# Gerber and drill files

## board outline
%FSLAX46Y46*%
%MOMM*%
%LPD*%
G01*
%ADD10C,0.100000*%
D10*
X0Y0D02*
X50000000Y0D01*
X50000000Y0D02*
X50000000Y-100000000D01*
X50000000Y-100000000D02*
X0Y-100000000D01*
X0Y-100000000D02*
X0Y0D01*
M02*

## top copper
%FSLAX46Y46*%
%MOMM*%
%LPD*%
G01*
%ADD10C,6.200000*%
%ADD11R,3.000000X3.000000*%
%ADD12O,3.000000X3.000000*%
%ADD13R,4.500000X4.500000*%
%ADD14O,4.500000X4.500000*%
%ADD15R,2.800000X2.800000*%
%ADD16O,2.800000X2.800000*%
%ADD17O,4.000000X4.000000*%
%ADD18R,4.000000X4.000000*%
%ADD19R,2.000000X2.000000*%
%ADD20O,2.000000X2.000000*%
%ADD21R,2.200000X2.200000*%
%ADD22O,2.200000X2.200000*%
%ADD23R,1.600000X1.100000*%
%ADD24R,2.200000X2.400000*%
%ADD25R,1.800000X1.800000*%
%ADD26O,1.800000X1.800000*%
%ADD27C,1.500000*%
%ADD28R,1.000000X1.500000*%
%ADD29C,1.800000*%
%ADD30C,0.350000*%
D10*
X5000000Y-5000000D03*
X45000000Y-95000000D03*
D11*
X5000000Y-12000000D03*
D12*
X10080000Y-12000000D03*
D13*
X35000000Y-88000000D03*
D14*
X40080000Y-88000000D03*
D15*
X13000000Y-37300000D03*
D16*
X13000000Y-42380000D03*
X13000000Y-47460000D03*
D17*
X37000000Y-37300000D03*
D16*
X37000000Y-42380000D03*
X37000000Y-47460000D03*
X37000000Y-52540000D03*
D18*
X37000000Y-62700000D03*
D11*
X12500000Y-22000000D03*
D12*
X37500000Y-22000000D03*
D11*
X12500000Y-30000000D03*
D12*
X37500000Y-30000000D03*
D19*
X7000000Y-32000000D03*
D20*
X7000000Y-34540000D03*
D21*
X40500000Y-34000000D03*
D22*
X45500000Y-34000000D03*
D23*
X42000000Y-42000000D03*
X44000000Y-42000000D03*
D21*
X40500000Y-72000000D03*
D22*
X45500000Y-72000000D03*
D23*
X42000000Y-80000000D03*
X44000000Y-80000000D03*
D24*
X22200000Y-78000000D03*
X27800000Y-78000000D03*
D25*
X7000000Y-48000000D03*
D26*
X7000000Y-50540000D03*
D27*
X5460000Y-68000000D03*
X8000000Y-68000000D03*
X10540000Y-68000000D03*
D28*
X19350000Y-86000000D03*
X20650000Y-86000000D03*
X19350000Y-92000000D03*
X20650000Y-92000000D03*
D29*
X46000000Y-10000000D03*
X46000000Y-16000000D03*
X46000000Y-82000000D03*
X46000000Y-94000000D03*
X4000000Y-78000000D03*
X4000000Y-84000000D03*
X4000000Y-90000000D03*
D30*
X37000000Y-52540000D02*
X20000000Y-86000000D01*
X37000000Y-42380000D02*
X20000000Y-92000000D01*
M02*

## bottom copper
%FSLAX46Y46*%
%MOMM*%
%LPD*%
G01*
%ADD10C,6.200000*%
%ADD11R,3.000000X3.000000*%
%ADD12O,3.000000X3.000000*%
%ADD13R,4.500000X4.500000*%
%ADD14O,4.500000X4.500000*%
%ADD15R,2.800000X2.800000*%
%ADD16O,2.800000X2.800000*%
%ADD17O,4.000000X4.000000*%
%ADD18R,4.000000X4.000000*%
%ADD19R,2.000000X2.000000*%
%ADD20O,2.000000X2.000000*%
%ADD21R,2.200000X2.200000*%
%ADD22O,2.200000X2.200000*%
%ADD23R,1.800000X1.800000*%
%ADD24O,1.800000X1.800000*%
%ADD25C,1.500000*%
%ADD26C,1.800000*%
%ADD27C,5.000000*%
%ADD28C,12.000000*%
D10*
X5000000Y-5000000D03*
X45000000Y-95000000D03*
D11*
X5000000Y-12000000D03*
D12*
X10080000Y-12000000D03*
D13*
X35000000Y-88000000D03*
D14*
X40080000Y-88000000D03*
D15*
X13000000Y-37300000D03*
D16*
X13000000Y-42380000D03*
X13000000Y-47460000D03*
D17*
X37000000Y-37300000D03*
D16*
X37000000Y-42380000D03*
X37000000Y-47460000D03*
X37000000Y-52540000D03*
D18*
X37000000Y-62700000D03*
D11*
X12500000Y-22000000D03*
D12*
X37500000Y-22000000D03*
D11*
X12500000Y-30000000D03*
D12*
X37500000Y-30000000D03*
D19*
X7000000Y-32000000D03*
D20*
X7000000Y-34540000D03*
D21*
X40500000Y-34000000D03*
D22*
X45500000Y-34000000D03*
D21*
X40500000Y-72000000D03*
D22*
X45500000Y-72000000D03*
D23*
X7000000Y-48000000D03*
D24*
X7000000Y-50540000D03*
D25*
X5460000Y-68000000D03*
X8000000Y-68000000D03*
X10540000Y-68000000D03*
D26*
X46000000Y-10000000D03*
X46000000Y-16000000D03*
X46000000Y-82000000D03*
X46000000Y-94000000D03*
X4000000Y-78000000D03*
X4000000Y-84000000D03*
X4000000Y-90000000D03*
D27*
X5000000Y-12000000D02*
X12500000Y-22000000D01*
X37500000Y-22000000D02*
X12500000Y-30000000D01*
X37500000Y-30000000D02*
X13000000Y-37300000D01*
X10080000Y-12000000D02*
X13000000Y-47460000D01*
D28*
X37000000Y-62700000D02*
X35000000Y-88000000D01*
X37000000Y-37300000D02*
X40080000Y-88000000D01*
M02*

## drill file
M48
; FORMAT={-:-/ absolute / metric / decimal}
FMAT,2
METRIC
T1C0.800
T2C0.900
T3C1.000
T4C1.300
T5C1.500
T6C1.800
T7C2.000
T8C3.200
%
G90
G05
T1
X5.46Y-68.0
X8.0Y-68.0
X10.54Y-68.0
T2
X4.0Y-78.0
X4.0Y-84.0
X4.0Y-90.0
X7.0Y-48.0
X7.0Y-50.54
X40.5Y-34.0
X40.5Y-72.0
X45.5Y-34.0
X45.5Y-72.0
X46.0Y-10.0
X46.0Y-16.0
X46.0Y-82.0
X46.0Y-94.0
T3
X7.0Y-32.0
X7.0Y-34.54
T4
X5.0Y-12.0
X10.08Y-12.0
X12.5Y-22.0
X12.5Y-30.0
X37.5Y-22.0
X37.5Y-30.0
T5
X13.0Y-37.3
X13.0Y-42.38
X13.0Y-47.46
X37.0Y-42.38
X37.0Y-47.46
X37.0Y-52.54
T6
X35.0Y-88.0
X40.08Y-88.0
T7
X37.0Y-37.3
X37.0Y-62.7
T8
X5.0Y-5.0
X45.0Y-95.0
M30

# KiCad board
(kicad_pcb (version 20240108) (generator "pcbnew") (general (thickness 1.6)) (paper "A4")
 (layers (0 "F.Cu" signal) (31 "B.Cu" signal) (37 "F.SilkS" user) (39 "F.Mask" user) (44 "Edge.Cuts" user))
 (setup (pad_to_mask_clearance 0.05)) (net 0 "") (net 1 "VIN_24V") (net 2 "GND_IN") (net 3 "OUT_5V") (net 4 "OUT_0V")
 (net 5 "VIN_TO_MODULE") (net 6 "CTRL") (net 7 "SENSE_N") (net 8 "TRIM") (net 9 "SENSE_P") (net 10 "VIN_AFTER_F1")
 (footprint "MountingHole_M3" (layer "F.Cu") (at 5 5)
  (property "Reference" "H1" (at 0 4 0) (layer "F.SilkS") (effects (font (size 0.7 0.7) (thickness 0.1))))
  (pad "1" np_thru_hole circle (at 0 0) (size 6.2 6.2) (drill 3.2) (layers "F.Cu" "B.Cu" "F.Mask" "B.Mask")))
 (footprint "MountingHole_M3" (layer "F.Cu") (at 45 95)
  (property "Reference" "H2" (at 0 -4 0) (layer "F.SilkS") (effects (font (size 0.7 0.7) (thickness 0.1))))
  (pad "1" np_thru_hole circle (at 0 0) (size 6.2 6.2) (drill 3.2) (layers "F.Cu" "B.Cu" "F.Mask" "B.Mask")))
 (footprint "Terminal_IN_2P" (layer "F.Cu") (at 5 12)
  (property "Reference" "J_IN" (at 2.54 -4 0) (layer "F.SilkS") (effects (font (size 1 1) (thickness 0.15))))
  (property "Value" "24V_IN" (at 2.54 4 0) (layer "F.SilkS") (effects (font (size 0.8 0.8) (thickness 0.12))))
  (pad "1" thru_hole rect (at 0 0) (size 3 3) (drill 1.3) (layers "F.Cu" "B.Cu" "F.Mask" "B.Mask") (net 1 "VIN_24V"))
  (pad "2" thru_hole oval (at 5.08 0) (size 3 3) (drill 1.3) (layers "F.Cu" "B.Cu" "F.Mask" "B.Mask") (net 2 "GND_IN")))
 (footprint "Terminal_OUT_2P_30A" (layer "F.Cu") (at 35 88)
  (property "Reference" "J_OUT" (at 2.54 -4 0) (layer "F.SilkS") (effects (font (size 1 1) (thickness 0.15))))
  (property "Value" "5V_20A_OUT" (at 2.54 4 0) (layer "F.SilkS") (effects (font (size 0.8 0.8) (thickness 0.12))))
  (pad "1" thru_hole rect (at 0 0) (size 4.5 4.5) (drill 1.8) (layers "F.Cu" "B.Cu" "F.Mask" "B.Mask") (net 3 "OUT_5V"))
  (pad "2" thru_hole oval (at 5.08 0) (size 4.5 4.5) (drill 1.8) (layers "F.Cu" "B.Cu" "F.Mask" "B.Mask") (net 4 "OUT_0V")))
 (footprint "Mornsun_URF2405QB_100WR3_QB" (layer "F.Cu") (at 25 50)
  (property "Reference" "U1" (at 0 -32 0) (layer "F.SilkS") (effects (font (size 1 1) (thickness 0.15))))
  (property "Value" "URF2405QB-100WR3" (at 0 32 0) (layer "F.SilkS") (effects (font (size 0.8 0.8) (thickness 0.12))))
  (pad "1" thru_hole rect (at -12 -12.7) (size 2.8 2.8) (drill 1.5) (layers "F.Cu" "B.Cu" "F.Mask" "B.Mask") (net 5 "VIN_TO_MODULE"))
  (pad "2" thru_hole oval (at -12 -7.62) (size 2.8 2.8) (drill 1.5) (layers "F.Cu" "B.Cu" "F.Mask" "B.Mask") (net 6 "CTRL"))
  (pad "3" thru_hole oval (at -12 -2.54) (size 2.8 2.8) (drill 1.5) (layers "F.Cu" "B.Cu" "F.Mask" "B.Mask") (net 2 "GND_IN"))
  (pad "4" thru_hole oval (at 12 -12.7) (size 4.0 4.0) (drill 2.0) (layers "F.Cu" "B.Cu" "F.Mask" "B.Mask") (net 4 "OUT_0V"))
  (pad "5" thru_hole oval (at 12 -7.62) (size 2.8 2.8) (drill 1.5) (layers "F.Cu" "B.Cu" "F.Mask" "B.Mask") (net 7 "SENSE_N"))
  (pad "6" thru_hole oval (at 12 -2.54) (size 2.8 2.8) (drill 1.5) (layers "F.Cu" "B.Cu" "F.Mask" "B.Mask") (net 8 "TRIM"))
  (pad "7" thru_hole oval (at 12 2.54) (size 2.8 2.8) (drill 1.5) (layers "F.Cu" "B.Cu" "F.Mask" "B.Mask") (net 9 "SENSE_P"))
  (pad "8" thru_hole rect (at 12 12.7) (size 4.0 4.0) (drill 2.0) (layers "F.Cu" "B.Cu" "F.Mask" "B.Mask") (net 3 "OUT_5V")))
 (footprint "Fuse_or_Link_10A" (layer "F.Cu") (at 25 22)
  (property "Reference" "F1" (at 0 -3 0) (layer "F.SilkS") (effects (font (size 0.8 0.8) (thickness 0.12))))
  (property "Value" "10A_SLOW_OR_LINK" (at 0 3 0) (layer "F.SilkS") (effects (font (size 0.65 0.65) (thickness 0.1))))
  (pad "1" thru_hole rect (at -12.5 0) (size 3 3) (drill 1.3) (layers "F.Cu" "B.Cu" "F.Mask" "B.Mask") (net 1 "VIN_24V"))
  (pad "2" thru_hole oval (at 12.5 0) (size 3 3) (drill 1.3) (layers "F.Cu" "B.Cu" "F.Mask" "B.Mask") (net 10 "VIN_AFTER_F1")))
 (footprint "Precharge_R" (layer "F.Cu") (at 25 30)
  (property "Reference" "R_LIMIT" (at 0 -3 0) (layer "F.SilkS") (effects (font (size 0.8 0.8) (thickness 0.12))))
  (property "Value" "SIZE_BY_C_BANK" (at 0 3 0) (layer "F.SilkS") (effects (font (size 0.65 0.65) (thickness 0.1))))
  (pad "1" thru_hole rect (at -12.5 0) (size 3 3) (drill 1.3) (layers "F.Cu" "B.Cu" "F.Mask" "B.Mask") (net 10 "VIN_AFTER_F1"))
  (pad "2" thru_hole oval (at 12.5 0) (size 3 3) (drill 1.3) (layers "F.Cu" "B.Cu" "F.Mask" "B.Mask") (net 5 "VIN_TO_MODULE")))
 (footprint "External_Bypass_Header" (layer "F.Cu") (at 7 32)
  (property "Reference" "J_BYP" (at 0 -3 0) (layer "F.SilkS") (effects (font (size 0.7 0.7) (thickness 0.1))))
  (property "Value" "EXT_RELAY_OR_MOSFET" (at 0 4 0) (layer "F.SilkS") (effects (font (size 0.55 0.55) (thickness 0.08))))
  (pad "1" thru_hole rect (at 0 0) (size 2 2) (drill 1.0) (layers "F.Cu" "B.Cu" "F.Mask" "B.Mask") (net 10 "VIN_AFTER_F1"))
  (pad "2" thru_hole oval (at 0 2.54) (size 2 2) (drill 1.0) (layers "F.Cu" "B.Cu" "F.Mask" "B.Mask") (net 5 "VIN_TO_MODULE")))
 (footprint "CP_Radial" (layer "F.Cu") (at 43 34)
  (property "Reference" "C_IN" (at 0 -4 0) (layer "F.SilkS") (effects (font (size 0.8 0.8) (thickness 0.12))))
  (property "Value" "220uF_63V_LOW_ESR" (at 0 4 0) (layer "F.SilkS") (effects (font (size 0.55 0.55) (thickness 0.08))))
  (pad "1" thru_hole rect (at -2.5 0) (size 2.2 2.2) (drill 0.9) (layers "F.Cu" "B.Cu" "F.Mask" "B.Mask") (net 5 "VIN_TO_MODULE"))
  (pad "2" thru_hole oval (at 2.5 0) (size 2.2 2.2) (drill 0.9) (layers "F.Cu" "B.Cu" "F.Mask" "B.Mask") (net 2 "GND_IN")))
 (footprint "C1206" (layer "F.Cu") (at 43 42)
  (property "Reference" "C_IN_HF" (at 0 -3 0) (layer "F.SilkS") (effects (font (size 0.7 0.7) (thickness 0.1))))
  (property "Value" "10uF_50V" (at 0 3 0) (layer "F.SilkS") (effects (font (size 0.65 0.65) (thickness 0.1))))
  (pad "1" smd rect (at -1 0) (size 1.6 1.1) (layers "F.Cu" "F.Mask") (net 5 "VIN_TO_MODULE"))
  (pad "2" smd rect (at 1 0) (size 1.6 1.1) (layers "F.Cu" "F.Mask") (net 2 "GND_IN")))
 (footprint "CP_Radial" (layer "F.Cu") (at 43 72)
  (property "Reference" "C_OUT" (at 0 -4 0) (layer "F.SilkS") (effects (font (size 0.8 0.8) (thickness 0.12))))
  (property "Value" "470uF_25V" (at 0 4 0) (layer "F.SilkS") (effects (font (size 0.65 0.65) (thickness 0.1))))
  (pad "1" thru_hole rect (at -2.5 0) (size 2.2 2.2) (drill 0.9) (layers "F.Cu" "B.Cu" "F.Mask" "B.Mask") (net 3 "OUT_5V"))
  (pad "2" thru_hole oval (at 2.5 0) (size 2.2 2.2) (drill 0.9) (layers "F.Cu" "B.Cu" "F.Mask" "B.Mask") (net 4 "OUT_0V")))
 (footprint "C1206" (layer "F.Cu") (at 43 80)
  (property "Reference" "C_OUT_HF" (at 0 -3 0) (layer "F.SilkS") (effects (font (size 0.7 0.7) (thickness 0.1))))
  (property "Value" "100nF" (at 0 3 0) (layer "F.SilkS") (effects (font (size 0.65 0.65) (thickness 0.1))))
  (pad "1" smd rect (at -1 0) (size 1.6 1.1) (layers "F.Cu" "F.Mask") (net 3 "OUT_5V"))
  (pad "2" smd rect (at 1 0) (size 1.6 1.1) (layers "F.Cu" "F.Mask") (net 4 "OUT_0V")))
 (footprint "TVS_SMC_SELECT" (layer "F.Cu") (at 25 78)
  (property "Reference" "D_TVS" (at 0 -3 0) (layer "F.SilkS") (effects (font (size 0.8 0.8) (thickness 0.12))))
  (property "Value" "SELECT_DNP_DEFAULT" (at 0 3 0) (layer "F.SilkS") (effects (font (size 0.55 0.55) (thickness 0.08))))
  (pad "1" smd rect (at -2.8 0) (size 2.2 2.4) (layers "F.Cu" "F.Mask") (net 3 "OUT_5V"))
  (pad "2" smd rect (at 2.8 0) (size 2.2 2.4) (layers "F.Cu" "F.Mask") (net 4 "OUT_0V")))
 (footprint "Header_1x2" (layer "F.Cu") (at 7 48)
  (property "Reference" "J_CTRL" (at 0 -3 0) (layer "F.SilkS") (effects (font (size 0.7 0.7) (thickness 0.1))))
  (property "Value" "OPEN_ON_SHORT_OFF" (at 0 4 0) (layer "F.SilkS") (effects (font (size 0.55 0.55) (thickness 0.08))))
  (pad "1" thru_hole rect (at 0 0) (size 1.8 1.8) (drill 0.9) (layers "F.Cu" "B.Cu" "F.Mask" "B.Mask") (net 6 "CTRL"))
  (pad "2" thru_hole oval (at 0 2.54) (size 1.8 1.8) (drill 0.9) (layers "F.Cu" "B.Cu" "F.Mask" "B.Mask") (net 2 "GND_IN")))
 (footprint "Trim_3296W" (layer "F.Cu") (at 8 68)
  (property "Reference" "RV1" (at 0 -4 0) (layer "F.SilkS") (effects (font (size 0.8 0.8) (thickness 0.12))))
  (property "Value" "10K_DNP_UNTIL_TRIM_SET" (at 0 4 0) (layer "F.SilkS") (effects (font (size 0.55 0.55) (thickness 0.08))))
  (pad "1" thru_hole circle (at -2.54 0) (size 1.5 1.5) (drill 0.8) (layers "F.Cu" "B.Cu" "F.Mask" "B.Mask") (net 7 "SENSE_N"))
  (pad "2" thru_hole circle (at 0 0) (size 1.5 1.5) (drill 0.8) (layers "F.Cu" "B.Cu" "F.Mask" "B.Mask") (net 8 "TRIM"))
  (pad "3" thru_hole circle (at 2.54 0) (size 1.5 1.5) (drill 0.8) (layers "F.Cu" "B.Cu" "F.Mask" "B.Mask") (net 9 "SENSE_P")))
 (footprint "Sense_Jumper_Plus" (layer "F.Cu") (at 20 86)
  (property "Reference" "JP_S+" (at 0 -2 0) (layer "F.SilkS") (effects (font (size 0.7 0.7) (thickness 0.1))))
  (pad "1" smd rect (at -0.65 0) (size 1.0 1.5) (layers "F.Cu" "F.Mask") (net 9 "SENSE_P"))
  (pad "2" smd rect (at 0.65 0) (size 1.0 1.5) (layers "F.Cu" "F.Mask") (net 3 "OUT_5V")))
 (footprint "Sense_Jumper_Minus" (layer "F.Cu") (at 20 92)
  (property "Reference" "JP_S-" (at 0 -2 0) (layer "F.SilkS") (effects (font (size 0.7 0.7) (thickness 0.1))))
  (pad "1" smd rect (at -0.65 0) (size 1.0 1.5) (layers "F.Cu" "F.Mask") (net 7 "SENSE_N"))
  (pad "2" smd rect (at 0.65 0) (size 1.0 1.5) (layers "F.Cu" "F.Mask") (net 4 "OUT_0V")))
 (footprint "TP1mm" (layer "F.Cu") (at 46 10)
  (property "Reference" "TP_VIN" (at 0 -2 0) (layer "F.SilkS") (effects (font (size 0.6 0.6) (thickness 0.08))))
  (pad "1" thru_hole circle (at 0 0) (size 1.8 1.8) (drill 0.9) (layers "F.Cu" "B.Cu" "F.Mask" "B.Mask") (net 1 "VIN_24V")))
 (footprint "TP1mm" (layer "F.Cu") (at 46 16)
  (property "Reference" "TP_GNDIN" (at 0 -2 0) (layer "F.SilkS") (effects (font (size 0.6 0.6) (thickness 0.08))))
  (pad "1" thru_hole circle (at 0 0) (size 1.8 1.8) (drill 0.9) (layers "F.Cu" "B.Cu" "F.Mask" "B.Mask") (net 2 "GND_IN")))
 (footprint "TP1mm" (layer "F.Cu") (at 46 82)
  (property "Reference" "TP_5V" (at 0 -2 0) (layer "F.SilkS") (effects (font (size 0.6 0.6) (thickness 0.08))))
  (pad "1" thru_hole circle (at 0 0) (size 1.8 1.8) (drill 0.9) (layers "F.Cu" "B.Cu" "F.Mask" "B.Mask") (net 3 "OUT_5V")))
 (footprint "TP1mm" (layer "F.Cu") (at 46 94)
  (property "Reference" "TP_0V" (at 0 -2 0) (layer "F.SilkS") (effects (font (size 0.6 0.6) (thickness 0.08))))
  (pad "1" thru_hole circle (at 0 0) (size 1.8 1.8) (drill 0.9) (layers "F.Cu" "B.Cu" "F.Mask" "B.Mask") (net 4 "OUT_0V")))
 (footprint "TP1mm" (layer "F.Cu") (at 4 78)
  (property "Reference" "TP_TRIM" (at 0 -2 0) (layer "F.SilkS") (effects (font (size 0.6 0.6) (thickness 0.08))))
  (pad "1" thru_hole circle (at 0 0) (size 1.8 1.8) (drill 0.9) (layers "F.Cu" "B.Cu" "F.Mask" "B.Mask") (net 8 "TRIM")))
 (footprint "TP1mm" (layer "F.Cu") (at 4 84)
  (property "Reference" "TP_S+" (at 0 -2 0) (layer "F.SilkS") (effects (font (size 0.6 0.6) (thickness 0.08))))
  (pad "1" thru_hole circle (at 0 0) (size 1.8 1.8) (drill 0.9) (layers "F.Cu" "B.Cu" "F.Mask" "B.Mask") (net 9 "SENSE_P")))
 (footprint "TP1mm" (layer "F.Cu") (at 4 90)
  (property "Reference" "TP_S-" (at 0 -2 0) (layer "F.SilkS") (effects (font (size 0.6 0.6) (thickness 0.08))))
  (pad "1" thru_hole circle (at 0 0) (size 1.8 1.8) (drill 0.9) (layers "F.Cu" "B.Cu" "F.Mask" "B.Mask") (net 7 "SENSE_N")))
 (segment (start 5 12) (end 12.5 22) (width 5.0) (layer "B.Cu") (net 1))
 (segment (start 37.5 22) (end 12.5 30) (width 5.0) (layer "B.Cu") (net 10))
 (segment (start 37.5 30) (end 13 37.3) (width 5.0) (layer "B.Cu") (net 5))
 (segment (start 10.08 12) (end 13 47.46) (width 5.0) (layer "B.Cu") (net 2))
 (segment (start 37 62.7) (end 35 88) (width 12.0) (layer "B.Cu") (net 3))
 (segment (start 37 37.3) (end 40.08 88) (width 12.0) (layer "B.Cu") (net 4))
 (segment (start 37 52.54) (end 20 86) (width 0.35) (layer "F.Cu") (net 9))
 (segment (start 37 42.38) (end 20 92) (width 0.35) (layer "F.Cu") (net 7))
 (gr_line (start 0 0) (end 50 0) (stroke (width 0.1) (type default)) (layer "Edge.Cuts"))
 (gr_line (start 50 0) (end 50 100) (stroke (width 0.1) (type default)) (layer "Edge.Cuts"))
 (gr_line (start 50 100) (end 0 100) (stroke (width 0.1) (type default)) (layer "Edge.Cuts"))
 (gr_line (start 0 100) (end 0 0) (stroke (width 0.1) (type default)) (layer "Edge.Cuts")))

